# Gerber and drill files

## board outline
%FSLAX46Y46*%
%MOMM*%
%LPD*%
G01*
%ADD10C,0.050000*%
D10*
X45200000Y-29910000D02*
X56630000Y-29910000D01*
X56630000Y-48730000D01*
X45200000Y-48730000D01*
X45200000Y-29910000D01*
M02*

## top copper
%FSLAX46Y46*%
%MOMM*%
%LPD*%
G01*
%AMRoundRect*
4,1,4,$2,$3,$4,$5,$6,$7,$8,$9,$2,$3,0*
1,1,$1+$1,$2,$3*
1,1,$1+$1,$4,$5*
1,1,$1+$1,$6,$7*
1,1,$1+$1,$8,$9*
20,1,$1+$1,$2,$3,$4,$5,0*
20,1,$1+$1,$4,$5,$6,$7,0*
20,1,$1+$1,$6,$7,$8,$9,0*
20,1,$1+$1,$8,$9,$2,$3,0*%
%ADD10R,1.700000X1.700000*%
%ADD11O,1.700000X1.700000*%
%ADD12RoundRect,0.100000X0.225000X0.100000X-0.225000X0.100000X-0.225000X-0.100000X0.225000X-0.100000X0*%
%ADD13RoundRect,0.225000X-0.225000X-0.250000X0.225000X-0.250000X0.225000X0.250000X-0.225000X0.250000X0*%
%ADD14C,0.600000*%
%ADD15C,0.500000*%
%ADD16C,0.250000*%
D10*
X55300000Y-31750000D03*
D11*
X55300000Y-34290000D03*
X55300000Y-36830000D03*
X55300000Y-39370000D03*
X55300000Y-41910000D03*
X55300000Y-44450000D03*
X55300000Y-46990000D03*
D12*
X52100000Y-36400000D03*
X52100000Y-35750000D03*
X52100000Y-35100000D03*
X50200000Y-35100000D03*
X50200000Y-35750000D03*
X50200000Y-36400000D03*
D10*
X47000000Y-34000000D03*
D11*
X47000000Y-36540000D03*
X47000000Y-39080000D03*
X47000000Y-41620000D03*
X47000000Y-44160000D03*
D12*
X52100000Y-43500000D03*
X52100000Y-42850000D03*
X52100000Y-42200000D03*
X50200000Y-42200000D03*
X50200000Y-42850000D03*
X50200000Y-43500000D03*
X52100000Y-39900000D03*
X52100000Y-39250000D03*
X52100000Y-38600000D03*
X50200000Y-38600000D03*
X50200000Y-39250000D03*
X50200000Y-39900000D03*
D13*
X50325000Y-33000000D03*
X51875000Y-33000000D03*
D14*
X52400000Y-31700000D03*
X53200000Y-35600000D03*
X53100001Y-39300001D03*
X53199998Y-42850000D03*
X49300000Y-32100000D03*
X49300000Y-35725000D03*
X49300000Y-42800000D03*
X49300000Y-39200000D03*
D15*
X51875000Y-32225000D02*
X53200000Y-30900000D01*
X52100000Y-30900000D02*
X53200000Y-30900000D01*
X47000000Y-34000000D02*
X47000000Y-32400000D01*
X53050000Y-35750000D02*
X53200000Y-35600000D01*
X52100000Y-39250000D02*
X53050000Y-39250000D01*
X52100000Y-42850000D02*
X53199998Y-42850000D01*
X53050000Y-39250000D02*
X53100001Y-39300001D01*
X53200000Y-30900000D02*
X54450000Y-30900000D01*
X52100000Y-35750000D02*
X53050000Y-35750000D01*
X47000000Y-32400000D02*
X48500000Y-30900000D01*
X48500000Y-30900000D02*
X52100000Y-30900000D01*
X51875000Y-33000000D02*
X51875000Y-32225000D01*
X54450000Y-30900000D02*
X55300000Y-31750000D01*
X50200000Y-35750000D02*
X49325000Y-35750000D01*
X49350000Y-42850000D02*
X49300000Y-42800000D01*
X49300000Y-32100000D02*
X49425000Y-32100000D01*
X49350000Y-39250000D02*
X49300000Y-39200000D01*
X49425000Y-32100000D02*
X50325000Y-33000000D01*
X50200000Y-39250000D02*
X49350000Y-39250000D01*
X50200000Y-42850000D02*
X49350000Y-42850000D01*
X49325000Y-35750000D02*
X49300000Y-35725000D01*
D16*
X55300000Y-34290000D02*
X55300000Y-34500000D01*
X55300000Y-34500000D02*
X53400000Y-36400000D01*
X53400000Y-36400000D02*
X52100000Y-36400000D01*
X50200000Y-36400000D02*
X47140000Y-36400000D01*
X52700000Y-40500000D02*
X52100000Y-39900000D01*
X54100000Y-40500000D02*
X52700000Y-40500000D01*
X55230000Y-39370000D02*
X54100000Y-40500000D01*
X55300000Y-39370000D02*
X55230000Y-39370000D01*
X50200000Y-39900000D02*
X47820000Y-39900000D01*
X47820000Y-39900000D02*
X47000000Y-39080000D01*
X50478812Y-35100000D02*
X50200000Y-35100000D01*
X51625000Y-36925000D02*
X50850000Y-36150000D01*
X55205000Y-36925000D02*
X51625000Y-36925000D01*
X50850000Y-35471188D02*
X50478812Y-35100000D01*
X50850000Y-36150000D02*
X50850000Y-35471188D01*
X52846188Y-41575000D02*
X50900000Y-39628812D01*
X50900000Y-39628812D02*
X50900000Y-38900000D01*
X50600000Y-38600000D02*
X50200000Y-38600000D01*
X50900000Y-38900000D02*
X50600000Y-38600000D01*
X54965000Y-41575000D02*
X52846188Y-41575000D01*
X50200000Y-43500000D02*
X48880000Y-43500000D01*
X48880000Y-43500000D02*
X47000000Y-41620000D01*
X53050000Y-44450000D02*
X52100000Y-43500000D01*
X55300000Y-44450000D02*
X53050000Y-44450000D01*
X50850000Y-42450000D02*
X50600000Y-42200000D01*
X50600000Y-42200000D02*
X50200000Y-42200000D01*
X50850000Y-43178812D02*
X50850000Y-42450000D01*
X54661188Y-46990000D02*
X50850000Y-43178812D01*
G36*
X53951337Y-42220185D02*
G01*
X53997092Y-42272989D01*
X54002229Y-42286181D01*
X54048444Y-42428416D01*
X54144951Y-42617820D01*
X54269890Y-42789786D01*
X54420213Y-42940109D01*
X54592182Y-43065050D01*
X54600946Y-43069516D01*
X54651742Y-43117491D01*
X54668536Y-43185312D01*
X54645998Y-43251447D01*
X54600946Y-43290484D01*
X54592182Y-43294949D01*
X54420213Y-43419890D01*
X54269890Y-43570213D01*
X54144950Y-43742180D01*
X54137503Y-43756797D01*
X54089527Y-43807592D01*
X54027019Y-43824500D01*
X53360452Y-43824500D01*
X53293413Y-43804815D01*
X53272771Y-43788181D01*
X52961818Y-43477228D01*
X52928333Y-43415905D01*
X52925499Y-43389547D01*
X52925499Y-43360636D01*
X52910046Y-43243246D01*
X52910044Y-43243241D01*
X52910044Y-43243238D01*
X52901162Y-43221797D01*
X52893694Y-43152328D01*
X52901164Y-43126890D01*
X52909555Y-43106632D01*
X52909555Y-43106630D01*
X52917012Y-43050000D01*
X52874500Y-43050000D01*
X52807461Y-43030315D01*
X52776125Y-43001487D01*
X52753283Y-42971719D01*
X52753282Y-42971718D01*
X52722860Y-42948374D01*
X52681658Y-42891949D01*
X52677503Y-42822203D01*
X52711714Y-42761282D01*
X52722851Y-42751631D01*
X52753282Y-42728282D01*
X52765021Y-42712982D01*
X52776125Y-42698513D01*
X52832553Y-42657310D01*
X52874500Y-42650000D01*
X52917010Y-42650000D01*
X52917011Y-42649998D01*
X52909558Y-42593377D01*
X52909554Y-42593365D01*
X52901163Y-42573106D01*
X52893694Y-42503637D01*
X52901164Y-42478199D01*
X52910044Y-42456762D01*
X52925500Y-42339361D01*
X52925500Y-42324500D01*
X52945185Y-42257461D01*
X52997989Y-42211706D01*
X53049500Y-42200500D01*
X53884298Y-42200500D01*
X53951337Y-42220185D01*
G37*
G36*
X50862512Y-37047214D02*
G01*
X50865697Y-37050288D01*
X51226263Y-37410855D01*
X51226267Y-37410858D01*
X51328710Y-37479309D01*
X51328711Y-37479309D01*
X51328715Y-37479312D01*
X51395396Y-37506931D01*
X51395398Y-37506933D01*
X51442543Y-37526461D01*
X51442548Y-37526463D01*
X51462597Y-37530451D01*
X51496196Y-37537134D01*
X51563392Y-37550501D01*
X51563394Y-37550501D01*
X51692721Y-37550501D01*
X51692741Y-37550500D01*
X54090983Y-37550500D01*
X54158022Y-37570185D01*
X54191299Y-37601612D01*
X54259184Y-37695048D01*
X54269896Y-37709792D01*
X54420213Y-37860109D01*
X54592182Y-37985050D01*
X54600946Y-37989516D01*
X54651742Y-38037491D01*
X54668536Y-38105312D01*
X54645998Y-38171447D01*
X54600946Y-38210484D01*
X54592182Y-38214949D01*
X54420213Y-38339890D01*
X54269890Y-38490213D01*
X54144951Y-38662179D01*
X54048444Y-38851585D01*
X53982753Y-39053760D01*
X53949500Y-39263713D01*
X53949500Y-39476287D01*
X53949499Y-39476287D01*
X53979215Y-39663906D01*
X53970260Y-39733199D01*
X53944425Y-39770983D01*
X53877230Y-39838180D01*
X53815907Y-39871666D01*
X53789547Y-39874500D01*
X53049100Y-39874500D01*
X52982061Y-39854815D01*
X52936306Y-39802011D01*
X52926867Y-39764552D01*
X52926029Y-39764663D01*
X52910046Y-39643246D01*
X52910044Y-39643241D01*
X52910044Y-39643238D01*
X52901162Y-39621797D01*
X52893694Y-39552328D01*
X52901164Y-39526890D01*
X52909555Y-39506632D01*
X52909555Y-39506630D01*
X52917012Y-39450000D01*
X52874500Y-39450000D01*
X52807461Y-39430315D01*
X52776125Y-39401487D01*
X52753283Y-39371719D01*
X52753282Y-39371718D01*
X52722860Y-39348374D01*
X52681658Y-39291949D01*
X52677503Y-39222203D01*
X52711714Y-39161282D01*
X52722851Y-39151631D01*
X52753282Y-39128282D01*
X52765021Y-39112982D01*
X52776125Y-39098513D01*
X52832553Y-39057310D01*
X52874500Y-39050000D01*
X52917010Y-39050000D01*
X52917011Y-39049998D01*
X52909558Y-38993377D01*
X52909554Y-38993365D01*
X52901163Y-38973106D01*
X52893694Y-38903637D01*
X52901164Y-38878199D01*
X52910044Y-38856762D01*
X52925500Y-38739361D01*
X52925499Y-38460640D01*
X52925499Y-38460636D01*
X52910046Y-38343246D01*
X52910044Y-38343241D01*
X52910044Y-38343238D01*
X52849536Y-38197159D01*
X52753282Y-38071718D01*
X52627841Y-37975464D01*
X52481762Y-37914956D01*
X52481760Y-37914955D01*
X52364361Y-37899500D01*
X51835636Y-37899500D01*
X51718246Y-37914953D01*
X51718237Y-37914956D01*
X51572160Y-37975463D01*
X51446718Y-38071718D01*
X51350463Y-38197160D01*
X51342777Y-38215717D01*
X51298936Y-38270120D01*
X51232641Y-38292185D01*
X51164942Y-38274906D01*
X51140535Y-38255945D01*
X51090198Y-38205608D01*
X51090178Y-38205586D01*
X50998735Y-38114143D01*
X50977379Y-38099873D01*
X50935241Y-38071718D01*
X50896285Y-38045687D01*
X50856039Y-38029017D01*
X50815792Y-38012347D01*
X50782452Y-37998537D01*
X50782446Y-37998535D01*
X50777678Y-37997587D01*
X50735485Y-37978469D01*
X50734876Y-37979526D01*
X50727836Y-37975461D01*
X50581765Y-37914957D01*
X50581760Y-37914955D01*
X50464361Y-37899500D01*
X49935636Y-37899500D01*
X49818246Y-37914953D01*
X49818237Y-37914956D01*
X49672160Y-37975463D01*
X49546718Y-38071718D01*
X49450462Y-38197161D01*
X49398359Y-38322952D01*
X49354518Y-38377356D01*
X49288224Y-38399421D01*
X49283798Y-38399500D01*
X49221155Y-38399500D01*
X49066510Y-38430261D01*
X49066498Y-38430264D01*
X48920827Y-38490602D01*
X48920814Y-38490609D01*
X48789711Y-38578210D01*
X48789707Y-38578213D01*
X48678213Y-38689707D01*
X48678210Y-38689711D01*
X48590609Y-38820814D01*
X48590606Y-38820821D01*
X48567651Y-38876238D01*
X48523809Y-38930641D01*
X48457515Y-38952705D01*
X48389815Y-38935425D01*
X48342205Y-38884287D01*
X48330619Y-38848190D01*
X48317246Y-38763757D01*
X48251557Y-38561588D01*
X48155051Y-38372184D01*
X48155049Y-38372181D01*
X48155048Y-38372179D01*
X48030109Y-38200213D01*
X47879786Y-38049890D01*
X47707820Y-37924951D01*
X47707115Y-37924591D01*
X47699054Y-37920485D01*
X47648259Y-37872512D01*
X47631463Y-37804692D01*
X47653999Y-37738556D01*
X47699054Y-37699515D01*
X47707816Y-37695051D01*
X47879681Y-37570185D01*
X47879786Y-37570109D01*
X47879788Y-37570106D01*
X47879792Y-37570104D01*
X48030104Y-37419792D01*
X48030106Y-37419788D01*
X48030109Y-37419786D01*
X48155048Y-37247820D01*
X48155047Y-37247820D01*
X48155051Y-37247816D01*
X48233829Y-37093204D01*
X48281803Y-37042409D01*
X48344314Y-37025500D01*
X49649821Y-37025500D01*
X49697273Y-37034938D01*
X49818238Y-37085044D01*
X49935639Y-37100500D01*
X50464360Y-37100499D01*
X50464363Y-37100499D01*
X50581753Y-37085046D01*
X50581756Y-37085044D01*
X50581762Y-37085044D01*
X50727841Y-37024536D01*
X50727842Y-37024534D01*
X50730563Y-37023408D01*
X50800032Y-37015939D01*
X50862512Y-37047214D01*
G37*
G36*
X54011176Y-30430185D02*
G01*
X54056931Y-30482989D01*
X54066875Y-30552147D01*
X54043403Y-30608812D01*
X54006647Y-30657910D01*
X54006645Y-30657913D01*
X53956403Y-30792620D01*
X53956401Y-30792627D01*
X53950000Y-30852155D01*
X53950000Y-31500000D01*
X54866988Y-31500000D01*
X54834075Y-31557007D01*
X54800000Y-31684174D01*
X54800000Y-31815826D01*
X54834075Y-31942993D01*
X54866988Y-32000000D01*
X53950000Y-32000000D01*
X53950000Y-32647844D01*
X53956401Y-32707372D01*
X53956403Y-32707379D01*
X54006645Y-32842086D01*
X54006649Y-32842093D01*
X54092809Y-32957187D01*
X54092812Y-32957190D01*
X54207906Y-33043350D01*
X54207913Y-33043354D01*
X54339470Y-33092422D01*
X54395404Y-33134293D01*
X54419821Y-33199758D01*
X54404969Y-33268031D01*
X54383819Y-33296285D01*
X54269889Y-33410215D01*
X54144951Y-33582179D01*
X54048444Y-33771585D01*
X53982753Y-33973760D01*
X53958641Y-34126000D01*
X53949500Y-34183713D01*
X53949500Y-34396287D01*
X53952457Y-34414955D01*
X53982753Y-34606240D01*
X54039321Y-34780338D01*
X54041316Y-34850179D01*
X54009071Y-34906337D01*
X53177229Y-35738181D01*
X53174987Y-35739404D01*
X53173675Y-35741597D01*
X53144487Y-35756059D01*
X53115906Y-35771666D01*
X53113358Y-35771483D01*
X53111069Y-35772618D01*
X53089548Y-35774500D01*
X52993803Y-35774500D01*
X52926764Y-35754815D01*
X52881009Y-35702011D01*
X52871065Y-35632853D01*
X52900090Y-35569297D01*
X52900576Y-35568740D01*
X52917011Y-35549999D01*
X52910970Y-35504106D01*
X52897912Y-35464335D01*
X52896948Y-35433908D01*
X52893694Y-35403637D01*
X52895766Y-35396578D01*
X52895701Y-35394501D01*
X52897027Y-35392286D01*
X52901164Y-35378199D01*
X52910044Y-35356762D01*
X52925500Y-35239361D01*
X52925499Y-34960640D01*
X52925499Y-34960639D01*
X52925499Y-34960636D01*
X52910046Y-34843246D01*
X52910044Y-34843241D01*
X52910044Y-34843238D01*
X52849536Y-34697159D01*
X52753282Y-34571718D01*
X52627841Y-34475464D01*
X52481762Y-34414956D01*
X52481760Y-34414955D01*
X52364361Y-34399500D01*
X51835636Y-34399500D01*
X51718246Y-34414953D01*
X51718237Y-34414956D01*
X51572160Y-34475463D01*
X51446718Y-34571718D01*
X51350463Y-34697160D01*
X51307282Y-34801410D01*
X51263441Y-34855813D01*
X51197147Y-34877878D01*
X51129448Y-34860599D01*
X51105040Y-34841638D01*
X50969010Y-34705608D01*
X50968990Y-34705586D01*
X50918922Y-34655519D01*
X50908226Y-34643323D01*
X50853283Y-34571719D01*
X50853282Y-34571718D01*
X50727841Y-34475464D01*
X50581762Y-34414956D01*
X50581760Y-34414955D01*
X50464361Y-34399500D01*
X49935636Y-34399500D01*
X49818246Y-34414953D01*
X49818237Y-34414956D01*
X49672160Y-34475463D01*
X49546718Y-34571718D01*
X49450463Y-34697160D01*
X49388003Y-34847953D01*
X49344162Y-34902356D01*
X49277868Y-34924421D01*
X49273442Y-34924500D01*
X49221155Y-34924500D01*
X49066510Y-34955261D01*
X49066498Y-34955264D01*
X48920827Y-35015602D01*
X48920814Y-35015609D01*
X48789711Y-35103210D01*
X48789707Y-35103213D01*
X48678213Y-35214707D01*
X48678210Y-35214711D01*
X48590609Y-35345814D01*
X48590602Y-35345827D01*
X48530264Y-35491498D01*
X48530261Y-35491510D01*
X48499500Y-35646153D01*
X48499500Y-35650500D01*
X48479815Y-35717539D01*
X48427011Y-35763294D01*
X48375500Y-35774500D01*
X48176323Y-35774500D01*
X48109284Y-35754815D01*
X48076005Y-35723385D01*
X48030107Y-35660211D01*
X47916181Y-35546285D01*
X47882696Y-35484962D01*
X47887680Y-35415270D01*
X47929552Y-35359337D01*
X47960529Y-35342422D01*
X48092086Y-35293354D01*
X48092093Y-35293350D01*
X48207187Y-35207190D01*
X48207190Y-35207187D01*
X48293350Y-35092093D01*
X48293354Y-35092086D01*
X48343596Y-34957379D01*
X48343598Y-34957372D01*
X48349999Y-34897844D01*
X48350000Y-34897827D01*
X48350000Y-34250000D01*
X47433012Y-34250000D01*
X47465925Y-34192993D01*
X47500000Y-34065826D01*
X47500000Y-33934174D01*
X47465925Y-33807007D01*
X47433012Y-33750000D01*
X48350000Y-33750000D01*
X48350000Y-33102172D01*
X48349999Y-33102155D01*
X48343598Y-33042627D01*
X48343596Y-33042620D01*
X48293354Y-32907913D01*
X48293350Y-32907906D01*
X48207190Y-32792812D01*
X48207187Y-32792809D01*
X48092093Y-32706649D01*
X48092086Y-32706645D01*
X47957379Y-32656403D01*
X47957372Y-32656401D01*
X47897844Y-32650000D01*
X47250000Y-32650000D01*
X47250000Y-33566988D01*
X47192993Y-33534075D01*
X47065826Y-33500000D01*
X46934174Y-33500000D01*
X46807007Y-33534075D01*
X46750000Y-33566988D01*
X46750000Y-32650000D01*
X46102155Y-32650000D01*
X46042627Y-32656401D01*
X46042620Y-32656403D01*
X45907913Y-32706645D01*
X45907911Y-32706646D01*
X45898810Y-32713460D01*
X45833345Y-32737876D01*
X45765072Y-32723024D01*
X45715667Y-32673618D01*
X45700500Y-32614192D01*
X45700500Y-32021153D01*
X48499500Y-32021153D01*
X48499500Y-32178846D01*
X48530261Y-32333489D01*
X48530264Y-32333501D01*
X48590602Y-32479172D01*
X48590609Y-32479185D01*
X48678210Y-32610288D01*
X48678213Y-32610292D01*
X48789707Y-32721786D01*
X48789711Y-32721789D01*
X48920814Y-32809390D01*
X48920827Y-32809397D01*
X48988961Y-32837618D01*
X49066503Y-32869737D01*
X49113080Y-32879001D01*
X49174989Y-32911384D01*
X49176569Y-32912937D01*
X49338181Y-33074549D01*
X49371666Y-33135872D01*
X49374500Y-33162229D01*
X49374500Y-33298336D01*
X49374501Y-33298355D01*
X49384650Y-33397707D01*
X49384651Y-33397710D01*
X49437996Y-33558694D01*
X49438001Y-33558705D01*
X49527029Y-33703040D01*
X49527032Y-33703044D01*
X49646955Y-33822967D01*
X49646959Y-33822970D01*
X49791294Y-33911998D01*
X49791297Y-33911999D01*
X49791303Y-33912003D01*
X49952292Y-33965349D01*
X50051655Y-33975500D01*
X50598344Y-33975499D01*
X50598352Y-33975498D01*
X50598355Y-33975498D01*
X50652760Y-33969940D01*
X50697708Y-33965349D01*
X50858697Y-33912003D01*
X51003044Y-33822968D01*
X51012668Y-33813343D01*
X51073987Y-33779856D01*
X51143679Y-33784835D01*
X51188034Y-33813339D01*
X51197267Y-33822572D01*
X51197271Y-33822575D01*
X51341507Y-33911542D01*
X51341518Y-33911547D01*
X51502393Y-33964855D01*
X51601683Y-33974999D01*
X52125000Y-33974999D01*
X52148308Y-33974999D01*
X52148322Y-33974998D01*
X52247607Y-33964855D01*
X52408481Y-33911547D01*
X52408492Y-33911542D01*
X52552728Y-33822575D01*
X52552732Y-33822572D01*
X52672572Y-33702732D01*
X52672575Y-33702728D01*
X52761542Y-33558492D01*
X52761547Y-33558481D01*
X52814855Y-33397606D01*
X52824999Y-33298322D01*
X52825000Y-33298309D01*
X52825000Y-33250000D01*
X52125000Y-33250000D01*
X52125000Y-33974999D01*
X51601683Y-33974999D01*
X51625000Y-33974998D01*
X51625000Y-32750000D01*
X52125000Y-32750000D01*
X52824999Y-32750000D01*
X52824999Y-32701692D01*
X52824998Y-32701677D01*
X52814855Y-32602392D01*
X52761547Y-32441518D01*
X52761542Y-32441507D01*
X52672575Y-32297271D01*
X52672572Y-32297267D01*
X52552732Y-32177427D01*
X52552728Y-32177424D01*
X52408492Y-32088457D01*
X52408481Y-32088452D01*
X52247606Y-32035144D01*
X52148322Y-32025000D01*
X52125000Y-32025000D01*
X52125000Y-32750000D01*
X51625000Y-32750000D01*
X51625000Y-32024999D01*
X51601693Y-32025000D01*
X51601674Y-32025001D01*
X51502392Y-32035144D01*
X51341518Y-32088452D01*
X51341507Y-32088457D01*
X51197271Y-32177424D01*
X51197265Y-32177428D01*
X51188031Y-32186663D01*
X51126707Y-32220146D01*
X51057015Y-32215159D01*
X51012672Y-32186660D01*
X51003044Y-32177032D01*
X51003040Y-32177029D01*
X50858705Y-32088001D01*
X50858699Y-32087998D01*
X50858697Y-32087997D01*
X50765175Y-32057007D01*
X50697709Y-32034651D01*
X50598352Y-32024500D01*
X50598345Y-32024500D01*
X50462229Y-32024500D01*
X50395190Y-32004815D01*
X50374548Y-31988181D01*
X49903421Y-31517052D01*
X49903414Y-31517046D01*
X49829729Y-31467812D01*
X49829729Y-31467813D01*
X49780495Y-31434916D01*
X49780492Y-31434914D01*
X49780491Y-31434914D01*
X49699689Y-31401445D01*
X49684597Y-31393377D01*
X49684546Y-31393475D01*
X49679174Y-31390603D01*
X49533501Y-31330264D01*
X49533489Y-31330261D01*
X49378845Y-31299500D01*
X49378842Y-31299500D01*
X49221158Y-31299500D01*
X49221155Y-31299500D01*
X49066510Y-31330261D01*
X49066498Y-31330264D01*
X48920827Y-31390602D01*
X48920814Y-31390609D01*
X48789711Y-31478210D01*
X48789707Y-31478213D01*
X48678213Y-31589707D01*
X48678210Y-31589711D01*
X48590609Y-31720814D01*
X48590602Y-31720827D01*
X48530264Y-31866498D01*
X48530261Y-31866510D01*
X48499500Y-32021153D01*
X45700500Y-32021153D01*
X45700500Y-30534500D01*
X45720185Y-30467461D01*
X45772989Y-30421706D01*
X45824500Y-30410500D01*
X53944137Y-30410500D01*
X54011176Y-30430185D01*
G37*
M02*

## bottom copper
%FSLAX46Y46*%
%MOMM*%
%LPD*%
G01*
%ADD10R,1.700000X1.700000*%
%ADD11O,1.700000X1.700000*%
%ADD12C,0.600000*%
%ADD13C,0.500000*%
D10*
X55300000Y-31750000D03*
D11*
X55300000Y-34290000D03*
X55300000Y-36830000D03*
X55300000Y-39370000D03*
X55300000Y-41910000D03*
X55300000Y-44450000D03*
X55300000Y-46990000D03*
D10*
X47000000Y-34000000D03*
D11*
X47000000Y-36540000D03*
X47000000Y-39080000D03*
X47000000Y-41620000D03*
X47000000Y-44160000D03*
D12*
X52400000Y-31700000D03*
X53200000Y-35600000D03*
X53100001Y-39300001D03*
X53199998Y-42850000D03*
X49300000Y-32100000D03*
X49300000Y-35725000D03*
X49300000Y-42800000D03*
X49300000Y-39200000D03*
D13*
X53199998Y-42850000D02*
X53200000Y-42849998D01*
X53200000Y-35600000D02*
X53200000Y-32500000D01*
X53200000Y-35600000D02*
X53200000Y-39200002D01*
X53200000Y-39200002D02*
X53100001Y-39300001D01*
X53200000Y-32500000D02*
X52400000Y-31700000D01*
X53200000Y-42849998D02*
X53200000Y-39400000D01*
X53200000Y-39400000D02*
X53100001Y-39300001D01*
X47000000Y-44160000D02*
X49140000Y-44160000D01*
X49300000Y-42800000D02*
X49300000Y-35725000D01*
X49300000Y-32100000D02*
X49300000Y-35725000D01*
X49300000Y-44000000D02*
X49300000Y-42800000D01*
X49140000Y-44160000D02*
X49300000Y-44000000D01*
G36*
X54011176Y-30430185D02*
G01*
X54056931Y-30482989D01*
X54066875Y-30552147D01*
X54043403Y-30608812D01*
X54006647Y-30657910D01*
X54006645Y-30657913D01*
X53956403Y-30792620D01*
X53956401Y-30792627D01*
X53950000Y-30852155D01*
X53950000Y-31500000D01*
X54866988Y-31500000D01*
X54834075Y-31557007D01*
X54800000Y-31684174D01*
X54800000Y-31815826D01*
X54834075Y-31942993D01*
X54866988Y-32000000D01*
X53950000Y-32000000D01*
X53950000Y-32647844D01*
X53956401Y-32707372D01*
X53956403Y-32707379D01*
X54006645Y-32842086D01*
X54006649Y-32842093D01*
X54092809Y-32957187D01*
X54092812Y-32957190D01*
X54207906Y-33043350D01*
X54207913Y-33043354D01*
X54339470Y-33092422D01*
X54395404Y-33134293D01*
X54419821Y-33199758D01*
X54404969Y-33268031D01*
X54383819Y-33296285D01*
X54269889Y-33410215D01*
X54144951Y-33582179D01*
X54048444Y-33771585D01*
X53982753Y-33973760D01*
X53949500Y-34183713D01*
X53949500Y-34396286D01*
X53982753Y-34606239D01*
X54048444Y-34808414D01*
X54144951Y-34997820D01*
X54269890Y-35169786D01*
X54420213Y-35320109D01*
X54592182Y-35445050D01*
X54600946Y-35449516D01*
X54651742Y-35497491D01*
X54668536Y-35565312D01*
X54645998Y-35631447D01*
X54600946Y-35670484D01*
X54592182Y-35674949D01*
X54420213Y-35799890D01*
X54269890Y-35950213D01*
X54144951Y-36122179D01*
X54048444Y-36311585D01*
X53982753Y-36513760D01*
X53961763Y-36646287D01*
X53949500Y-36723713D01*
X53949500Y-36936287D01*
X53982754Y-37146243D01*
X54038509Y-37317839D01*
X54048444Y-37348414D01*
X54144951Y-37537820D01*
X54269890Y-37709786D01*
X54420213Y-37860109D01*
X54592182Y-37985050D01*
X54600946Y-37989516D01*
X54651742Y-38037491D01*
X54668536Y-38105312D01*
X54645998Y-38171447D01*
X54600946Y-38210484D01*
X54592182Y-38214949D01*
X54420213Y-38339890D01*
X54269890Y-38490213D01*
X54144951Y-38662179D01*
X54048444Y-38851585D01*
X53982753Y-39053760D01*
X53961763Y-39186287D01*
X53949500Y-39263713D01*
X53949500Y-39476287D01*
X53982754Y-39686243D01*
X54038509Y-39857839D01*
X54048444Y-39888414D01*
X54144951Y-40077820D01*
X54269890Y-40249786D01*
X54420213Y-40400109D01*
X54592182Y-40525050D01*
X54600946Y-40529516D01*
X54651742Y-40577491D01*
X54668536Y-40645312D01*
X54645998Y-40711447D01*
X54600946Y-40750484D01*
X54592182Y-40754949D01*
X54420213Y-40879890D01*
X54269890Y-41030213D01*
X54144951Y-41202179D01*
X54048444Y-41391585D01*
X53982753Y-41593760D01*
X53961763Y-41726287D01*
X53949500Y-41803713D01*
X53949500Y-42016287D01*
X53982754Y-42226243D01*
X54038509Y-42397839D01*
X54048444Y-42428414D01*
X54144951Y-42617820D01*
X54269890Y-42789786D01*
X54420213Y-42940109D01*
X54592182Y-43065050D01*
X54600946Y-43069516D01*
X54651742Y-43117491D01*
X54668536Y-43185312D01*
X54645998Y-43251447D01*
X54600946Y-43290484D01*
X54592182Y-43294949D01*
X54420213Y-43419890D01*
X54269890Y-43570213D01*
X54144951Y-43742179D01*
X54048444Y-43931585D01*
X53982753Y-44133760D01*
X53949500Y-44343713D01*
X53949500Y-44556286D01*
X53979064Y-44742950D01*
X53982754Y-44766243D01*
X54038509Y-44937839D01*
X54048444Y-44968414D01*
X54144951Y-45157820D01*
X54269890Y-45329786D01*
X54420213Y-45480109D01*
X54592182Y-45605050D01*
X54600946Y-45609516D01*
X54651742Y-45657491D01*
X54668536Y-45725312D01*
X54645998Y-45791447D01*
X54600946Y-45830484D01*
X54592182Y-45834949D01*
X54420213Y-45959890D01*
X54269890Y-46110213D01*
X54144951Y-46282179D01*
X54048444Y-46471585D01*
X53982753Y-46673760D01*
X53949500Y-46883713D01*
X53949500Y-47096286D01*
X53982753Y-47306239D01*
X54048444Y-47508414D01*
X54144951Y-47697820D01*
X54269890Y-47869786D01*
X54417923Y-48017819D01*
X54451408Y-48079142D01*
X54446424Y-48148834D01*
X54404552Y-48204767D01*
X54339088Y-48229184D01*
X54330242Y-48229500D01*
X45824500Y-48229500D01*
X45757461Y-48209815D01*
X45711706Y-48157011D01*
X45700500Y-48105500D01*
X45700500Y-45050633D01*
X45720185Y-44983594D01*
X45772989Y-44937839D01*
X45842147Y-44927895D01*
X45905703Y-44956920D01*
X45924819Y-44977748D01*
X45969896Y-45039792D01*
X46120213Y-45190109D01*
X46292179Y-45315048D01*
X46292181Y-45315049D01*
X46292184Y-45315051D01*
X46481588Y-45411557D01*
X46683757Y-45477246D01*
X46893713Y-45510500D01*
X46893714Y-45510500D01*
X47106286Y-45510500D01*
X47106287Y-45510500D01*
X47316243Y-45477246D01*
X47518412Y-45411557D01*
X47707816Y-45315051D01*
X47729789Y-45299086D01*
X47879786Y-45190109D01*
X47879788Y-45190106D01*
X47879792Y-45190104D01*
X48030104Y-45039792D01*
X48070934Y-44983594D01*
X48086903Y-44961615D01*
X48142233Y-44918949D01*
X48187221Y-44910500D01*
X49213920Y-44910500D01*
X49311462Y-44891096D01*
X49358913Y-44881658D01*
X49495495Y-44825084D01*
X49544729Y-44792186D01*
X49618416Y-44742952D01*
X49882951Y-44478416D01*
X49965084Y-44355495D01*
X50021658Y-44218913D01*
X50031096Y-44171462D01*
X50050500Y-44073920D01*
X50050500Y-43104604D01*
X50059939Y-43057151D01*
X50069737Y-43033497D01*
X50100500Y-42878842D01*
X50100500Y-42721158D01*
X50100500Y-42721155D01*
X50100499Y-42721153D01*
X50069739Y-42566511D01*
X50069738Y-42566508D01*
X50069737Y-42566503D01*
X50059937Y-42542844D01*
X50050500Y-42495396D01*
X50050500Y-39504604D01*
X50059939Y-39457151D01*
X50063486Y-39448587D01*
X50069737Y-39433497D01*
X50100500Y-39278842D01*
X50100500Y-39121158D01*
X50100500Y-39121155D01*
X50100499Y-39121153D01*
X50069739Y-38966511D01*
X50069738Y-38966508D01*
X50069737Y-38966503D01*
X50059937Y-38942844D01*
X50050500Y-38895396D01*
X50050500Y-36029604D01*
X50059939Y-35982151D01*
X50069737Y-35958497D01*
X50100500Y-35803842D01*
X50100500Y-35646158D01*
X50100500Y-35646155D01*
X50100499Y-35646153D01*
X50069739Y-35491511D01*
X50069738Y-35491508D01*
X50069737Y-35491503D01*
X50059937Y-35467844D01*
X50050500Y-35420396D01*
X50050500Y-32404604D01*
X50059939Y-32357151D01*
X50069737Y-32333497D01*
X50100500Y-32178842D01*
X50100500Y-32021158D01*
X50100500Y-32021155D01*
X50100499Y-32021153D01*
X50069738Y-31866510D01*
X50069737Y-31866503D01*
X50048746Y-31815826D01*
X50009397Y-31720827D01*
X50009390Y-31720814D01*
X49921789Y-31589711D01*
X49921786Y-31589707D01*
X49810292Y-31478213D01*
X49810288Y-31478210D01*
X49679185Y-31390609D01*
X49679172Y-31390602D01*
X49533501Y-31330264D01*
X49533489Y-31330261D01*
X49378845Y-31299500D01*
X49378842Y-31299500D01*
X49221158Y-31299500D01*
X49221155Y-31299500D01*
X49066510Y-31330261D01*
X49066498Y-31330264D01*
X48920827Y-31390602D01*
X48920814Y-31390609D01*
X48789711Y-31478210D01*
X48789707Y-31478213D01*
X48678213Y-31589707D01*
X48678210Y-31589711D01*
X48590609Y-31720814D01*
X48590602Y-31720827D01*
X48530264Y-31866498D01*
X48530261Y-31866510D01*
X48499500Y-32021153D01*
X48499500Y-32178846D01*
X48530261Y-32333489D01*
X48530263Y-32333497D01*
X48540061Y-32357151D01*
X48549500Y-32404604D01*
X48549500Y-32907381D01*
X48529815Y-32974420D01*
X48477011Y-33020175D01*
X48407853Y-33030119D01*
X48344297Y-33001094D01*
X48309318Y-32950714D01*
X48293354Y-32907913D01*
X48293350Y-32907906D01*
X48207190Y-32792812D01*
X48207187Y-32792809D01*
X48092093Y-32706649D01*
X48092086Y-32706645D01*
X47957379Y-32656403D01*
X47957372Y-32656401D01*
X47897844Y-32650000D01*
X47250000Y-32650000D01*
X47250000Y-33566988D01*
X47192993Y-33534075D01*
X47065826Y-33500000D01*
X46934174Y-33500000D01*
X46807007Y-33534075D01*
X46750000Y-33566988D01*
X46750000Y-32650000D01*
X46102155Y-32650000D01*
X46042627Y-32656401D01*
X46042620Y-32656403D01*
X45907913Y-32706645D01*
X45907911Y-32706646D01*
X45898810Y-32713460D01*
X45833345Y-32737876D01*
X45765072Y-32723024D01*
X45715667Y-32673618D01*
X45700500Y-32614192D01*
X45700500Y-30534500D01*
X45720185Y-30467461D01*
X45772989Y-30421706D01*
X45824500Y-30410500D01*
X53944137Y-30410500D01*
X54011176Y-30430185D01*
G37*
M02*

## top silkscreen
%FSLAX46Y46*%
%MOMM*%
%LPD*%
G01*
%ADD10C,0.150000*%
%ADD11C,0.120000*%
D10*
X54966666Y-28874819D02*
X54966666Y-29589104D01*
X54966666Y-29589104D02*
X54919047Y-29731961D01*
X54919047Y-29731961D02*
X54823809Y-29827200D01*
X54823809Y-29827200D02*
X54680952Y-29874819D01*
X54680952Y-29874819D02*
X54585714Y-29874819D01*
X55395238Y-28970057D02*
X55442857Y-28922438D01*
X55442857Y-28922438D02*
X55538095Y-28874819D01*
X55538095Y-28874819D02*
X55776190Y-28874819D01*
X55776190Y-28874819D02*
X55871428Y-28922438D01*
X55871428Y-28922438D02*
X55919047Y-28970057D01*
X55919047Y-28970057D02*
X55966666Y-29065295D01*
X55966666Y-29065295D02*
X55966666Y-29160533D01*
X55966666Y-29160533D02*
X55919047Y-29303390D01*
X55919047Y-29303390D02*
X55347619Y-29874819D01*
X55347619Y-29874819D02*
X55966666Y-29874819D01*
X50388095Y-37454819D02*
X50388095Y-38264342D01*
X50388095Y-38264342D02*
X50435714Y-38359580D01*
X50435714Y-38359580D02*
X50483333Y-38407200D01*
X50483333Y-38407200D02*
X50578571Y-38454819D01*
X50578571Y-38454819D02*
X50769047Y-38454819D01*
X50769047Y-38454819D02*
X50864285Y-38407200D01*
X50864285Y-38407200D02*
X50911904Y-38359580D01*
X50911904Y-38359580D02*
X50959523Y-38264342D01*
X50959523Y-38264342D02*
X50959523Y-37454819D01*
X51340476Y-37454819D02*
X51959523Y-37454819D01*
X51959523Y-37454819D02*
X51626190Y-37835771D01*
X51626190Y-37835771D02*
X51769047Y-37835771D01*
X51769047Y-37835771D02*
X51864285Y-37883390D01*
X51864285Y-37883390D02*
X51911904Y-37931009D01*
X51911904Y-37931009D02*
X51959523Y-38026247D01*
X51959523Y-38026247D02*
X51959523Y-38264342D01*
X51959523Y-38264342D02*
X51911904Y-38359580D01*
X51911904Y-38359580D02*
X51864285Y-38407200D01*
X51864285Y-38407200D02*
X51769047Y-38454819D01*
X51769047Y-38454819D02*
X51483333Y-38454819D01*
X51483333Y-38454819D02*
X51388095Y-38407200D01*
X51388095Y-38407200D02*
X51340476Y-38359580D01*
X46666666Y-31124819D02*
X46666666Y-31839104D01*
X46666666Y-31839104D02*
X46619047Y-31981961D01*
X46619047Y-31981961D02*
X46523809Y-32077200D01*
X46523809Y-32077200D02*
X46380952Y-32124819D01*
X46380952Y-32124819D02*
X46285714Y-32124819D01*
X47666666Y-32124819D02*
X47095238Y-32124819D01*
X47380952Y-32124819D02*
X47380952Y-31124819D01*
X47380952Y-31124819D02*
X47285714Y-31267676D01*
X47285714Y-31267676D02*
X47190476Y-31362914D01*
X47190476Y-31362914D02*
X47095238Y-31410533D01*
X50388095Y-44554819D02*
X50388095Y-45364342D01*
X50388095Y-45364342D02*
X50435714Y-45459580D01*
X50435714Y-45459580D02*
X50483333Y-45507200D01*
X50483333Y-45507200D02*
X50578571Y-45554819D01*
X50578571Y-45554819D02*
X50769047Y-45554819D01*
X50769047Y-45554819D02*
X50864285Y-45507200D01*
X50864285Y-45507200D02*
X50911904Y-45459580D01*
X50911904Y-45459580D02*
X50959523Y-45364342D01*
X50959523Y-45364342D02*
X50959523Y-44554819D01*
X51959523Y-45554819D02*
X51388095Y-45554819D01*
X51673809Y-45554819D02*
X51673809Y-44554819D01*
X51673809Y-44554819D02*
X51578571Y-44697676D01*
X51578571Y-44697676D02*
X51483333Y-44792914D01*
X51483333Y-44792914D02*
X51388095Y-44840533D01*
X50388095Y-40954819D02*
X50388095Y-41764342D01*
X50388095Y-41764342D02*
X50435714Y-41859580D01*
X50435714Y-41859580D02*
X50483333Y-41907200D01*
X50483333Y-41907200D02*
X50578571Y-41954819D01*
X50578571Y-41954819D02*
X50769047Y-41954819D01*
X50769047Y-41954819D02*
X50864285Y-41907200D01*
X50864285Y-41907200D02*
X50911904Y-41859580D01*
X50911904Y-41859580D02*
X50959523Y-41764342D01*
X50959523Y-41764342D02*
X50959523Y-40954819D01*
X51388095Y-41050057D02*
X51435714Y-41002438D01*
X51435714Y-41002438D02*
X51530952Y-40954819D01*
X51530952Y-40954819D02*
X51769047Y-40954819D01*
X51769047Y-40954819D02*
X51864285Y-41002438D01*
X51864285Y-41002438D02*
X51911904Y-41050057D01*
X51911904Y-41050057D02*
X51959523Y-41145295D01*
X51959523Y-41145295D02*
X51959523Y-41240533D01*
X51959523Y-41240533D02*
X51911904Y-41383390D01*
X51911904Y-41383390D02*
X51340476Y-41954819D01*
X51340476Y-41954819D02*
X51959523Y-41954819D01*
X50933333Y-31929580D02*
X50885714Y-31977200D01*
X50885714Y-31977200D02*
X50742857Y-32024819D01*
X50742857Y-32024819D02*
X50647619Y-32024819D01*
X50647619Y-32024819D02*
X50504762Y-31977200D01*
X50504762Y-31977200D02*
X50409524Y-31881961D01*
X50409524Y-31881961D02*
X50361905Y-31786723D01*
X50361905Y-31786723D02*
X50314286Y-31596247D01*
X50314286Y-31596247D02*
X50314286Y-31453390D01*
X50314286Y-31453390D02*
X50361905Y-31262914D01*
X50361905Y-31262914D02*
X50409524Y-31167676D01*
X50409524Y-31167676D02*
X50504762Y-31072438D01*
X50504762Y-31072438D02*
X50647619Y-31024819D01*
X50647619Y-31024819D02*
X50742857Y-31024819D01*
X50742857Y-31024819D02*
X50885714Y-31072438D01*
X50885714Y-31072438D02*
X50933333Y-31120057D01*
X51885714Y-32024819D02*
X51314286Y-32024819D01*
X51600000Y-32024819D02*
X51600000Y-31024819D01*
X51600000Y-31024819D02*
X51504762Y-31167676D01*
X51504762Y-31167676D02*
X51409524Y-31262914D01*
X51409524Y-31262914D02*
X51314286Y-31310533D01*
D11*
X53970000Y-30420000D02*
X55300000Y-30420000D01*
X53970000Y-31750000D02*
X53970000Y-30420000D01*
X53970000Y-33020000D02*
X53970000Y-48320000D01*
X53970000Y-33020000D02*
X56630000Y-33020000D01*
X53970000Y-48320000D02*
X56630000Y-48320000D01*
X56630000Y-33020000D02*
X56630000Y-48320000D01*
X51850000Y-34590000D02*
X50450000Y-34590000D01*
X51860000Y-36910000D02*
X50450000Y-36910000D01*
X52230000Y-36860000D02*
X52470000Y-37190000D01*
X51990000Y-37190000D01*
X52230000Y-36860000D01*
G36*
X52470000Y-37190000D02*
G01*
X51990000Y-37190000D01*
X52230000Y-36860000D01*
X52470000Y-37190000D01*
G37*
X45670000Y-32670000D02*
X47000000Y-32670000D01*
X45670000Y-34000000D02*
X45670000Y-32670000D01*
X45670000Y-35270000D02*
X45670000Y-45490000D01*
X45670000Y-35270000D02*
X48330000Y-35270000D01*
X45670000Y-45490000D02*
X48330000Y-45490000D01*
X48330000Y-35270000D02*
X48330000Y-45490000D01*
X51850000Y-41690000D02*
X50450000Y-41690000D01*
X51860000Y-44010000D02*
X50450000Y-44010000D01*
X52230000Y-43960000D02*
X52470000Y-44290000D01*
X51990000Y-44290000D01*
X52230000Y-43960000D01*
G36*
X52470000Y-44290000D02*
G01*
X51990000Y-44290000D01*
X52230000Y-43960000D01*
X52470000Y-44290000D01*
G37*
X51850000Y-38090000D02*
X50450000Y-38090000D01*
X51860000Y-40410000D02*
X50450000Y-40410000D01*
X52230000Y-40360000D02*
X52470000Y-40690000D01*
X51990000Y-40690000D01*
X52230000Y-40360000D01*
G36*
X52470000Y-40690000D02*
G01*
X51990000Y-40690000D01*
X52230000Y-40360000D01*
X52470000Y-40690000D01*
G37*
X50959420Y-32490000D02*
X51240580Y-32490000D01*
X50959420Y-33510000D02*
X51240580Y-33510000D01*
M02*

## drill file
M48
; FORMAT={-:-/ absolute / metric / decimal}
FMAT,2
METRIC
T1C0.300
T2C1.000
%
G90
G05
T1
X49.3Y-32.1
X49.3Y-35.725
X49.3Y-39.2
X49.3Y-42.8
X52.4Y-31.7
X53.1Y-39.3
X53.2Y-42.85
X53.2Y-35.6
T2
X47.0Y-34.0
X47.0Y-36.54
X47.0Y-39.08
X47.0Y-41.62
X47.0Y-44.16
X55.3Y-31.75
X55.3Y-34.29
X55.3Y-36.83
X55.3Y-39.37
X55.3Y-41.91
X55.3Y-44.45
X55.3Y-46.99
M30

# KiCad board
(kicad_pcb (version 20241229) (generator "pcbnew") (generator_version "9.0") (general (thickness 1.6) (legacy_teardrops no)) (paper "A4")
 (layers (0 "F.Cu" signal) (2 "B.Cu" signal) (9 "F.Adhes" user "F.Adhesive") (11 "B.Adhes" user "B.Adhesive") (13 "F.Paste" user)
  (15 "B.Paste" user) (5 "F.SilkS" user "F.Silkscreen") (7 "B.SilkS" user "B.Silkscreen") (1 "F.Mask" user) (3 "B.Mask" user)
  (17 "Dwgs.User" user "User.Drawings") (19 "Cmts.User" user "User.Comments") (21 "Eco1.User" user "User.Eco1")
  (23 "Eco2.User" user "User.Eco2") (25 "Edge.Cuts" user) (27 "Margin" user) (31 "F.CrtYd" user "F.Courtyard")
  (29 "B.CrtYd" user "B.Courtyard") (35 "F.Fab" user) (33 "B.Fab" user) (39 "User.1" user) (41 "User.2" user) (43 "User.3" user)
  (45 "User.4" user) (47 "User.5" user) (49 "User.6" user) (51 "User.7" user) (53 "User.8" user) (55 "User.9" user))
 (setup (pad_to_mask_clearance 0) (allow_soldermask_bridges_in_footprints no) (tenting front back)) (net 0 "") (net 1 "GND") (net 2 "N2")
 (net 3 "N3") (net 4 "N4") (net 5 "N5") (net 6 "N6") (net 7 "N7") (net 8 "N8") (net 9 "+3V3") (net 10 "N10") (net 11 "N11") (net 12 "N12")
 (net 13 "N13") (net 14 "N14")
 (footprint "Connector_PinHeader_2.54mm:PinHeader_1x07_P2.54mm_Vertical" (layer "F.Cu") (at 55.3 31.75)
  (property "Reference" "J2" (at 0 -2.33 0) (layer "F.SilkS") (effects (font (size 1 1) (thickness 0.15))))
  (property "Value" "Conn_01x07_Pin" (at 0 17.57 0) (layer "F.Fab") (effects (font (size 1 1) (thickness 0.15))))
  (fp_line (start -1.33 -1.33) (end 0 -1.33) (stroke (width 0.12) (type solid)) (layer "F.SilkS"))
  (fp_line (start -1.33 0) (end -1.33 -1.33) (stroke (width 0.12) (type solid)) (layer "F.SilkS"))
  (fp_line (start -1.33 1.27) (end -1.33 16.57) (stroke (width 0.12) (type solid)) (layer "F.SilkS"))
  (fp_line (start -1.33 1.27) (end 1.33 1.27) (stroke (width 0.12) (type solid)) (layer "F.SilkS"))
  (fp_line (start -1.33 16.57) (end 1.33 16.57) (stroke (width 0.12) (type solid)) (layer "F.SilkS"))
  (fp_line (start 1.33 1.27) (end 1.33 16.57) (stroke (width 0.12) (type solid)) (layer "F.SilkS"))
  (pad "1" thru_hole rect (at 0 0) (size 1.7 1.7) (drill 1) (layers "*.Cu" "*.Mask") (remove_unused_layers no) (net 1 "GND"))
  (pad "2" thru_hole oval (at 0 2.54) (size 1.7 1.7) (drill 1) (layers "*.Cu" "*.Mask") (remove_unused_layers no) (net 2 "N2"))
  (pad "3" thru_hole oval (at 0 5.08) (size 1.7 1.7) (drill 1) (layers "*.Cu" "*.Mask") (remove_unused_layers no) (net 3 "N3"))
  (pad "4" thru_hole oval (at 0 7.62) (size 1.7 1.7) (drill 1) (layers "*.Cu" "*.Mask") (remove_unused_layers no) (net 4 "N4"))
  (pad "5" thru_hole oval (at 0 10.16) (size 1.7 1.7) (drill 1) (layers "*.Cu" "*.Mask") (remove_unused_layers no) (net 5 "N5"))
  (pad "6" thru_hole oval (at 0 12.7) (size 1.7 1.7) (drill 1) (layers "*.Cu" "*.Mask") (remove_unused_layers no) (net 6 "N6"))
  (pad "7" thru_hole oval (at 0 15.24) (size 1.7 1.7) (drill 1) (layers "*.Cu" "*.Mask") (remove_unused_layers no) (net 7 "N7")))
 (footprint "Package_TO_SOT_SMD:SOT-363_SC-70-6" (layer "F.Cu") (at 51.15 35.75 180)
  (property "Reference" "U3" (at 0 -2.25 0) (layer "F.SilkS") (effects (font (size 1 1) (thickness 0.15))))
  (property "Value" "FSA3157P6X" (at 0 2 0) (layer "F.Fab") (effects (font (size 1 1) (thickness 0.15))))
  (fp_line (start -0.7 1.16) (end 0.7 1.16) (stroke (width 0.12) (type solid)) (layer "F.SilkS"))
  (fp_line (start -0.71 -1.16) (end 0.7 -1.16) (stroke (width 0.12) (type solid)) (layer "F.SilkS"))
  (fp_poly
   (pts (xy -1.08 -1.11) (xy -1.32 -1.44) (xy -0.84 -1.44) (xy -1.08 -1.11)) (stroke (width 0.12) (type solid)) (fill yes) (layer "F.SilkS"))
  (pad "1" smd roundrect (at -0.95 -0.65 180) (size 0.65 0.4) (layers "F.Cu" "F.Mask" "F.Paste") (roundrect_rratio 0.25) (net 2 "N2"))
  (pad "2" smd roundrect (at -0.95 0 180) (size 0.65 0.4) (layers "F.Cu" "F.Mask" "F.Paste") (roundrect_rratio 0.25) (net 1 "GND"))
  (pad "3" smd roundrect (at -0.95 0.65 180) (size 0.65 0.4) (layers "F.Cu" "F.Mask" "F.Paste") (roundrect_rratio 0.25) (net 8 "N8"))
  (pad "4" smd roundrect (at 0.95 0.65 180) (size 0.65 0.4) (layers "F.Cu" "F.Mask" "F.Paste") (roundrect_rratio 0.25) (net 3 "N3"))
  (pad "5" smd roundrect (at 0.95 0 180) (size 0.65 0.4) (layers "F.Cu" "F.Mask" "F.Paste") (roundrect_rratio 0.25) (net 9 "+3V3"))
  (pad "6" smd roundrect (at 0.95 -0.65 180) (size 0.65 0.4) (layers "F.Cu" "F.Mask" "F.Paste") (roundrect_rratio 0.25) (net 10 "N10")))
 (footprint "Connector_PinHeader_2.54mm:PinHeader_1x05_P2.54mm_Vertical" (layer "F.Cu") (at 47 34)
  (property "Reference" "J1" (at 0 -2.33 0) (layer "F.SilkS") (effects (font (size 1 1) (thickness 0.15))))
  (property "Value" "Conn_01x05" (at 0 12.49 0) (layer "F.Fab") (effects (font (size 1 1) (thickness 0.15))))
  (fp_line (start -1.33 -1.33) (end 0 -1.33) (stroke (width 0.12) (type solid)) (layer "F.SilkS"))
  (fp_line (start -1.33 0) (end -1.33 -1.33) (stroke (width 0.12) (type solid)) (layer "F.SilkS"))
  (fp_line (start -1.33 1.27) (end -1.33 11.49) (stroke (width 0.12) (type solid)) (layer "F.SilkS"))
  (fp_line (start -1.33 1.27) (end 1.33 1.27) (stroke (width 0.12) (type solid)) (layer "F.SilkS"))
  (fp_line (start -1.33 11.49) (end 1.33 11.49) (stroke (width 0.12) (type solid)) (layer "F.SilkS"))
  (fp_line (start 1.33 1.27) (end 1.33 11.49) (stroke (width 0.12) (type solid)) (layer "F.SilkS"))
  (pad "1" thru_hole rect (at 0 0) (size 1.7 1.7) (drill 1) (layers "*.Cu" "*.Mask") (remove_unused_layers no) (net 1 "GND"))
  (pad "2" thru_hole oval (at 0 2.54) (size 1.7 1.7) (drill 1) (layers "*.Cu" "*.Mask") (remove_unused_layers no) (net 10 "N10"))
  (pad "3" thru_hole oval (at 0 5.08) (size 1.7 1.7) (drill 1) (layers "*.Cu" "*.Mask") (remove_unused_layers no) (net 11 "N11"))
  (pad "4" thru_hole oval (at 0 7.62) (size 1.7 1.7) (drill 1) (layers "*.Cu" "*.Mask") (remove_unused_layers no) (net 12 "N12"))
  (pad "5" thru_hole oval (at 0 10.16) (size 1.7 1.7) (drill 1) (layers "*.Cu" "*.Mask") (remove_unused_layers no) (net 9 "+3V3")))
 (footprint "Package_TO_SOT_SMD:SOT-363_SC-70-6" (layer "F.Cu") (at 51.15 42.85 180)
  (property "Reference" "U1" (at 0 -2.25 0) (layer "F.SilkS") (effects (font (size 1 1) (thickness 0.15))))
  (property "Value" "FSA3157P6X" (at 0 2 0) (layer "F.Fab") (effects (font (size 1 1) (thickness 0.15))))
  (fp_line (start -0.7 1.16) (end 0.7 1.16) (stroke (width 0.12) (type solid)) (layer "F.SilkS"))
  (fp_line (start -0.71 -1.16) (end 0.7 -1.16) (stroke (width 0.12) (type solid)) (layer "F.SilkS"))
  (fp_poly
   (pts (xy -1.08 -1.11) (xy -1.32 -1.44) (xy -0.84 -1.44) (xy -1.08 -1.11)) (stroke (width 0.12) (type solid)) (fill yes) (layer "F.SilkS"))
  (pad "1" smd roundrect (at -0.95 -0.65 180) (size 0.65 0.4) (layers "F.Cu" "F.Mask" "F.Paste") (roundrect_rratio 0.25) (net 6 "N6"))
  (pad "2" smd roundrect (at -0.95 0 180) (size 0.65 0.4) (layers "F.Cu" "F.Mask" "F.Paste") (roundrect_rratio 0.25) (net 1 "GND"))
  (pad "3" smd roundrect (at -0.95 0.65 180) (size 0.65 0.4) (layers "F.Cu" "F.Mask" "F.Paste") (roundrect_rratio 0.25) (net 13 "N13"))
  (pad "4" smd roundrect (at 0.95 0.65 180) (size 0.65 0.4) (layers "F.Cu" "F.Mask" "F.Paste") (roundrect_rratio 0.25) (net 7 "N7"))
  (pad "5" smd roundrect (at 0.95 0 180) (size 0.65 0.4) (layers "F.Cu" "F.Mask" "F.Paste") (roundrect_rratio 0.25) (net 9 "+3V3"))
  (pad "6" smd roundrect (at 0.95 -0.65 180) (size 0.65 0.4) (layers "F.Cu" "F.Mask" "F.Paste") (roundrect_rratio 0.25) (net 12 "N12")))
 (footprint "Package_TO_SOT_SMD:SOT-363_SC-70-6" (layer "F.Cu") (at 51.15 39.25 180)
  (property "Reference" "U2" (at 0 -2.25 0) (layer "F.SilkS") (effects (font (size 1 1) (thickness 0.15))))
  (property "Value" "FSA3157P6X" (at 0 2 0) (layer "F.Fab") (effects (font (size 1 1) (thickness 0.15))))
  (fp_line (start -0.7 1.16) (end 0.7 1.16) (stroke (width 0.12) (type solid)) (layer "F.SilkS"))
  (fp_line (start -0.71 -1.16) (end 0.7 -1.16) (stroke (width 0.12) (type solid)) (layer "F.SilkS"))
  (fp_poly
   (pts (xy -1.08 -1.11) (xy -1.32 -1.44) (xy -0.84 -1.44) (xy -1.08 -1.11)) (stroke (width 0.12) (type solid)) (fill yes) (layer "F.SilkS"))
  (pad "1" smd roundrect (at -0.95 -0.65 180) (size 0.65 0.4) (layers "F.Cu" "F.Mask" "F.Paste") (roundrect_rratio 0.25) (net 4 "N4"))
  (pad "2" smd roundrect (at -0.95 0 180) (size 0.65 0.4) (layers "F.Cu" "F.Mask" "F.Paste") (roundrect_rratio 0.25) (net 1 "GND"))
  (pad "3" smd roundrect (at -0.95 0.65 180) (size 0.65 0.4) (layers "F.Cu" "F.Mask" "F.Paste") (roundrect_rratio 0.25) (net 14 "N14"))
  (pad "4" smd roundrect (at 0.95 0.65 180) (size 0.65 0.4) (layers "F.Cu" "F.Mask" "F.Paste") (roundrect_rratio 0.25) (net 5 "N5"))
  (pad "5" smd roundrect (at 0.95 0 180) (size 0.65 0.4) (layers "F.Cu" "F.Mask" "F.Paste") (roundrect_rratio 0.25) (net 9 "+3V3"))
  (pad "6" smd roundrect (at 0.95 -0.65 180) (size 0.65 0.4) (layers "F.Cu" "F.Mask" "F.Paste") (roundrect_rratio 0.25) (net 11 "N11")))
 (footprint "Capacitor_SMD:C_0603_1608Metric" (layer "F.Cu") (at 51.1 33)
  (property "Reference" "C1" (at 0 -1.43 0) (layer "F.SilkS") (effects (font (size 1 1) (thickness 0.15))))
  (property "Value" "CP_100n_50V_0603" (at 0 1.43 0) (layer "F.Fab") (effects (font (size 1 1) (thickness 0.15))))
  (fp_line (start -0.14058 -0.51) (end 0.14058 -0.51) (stroke (width 0.12) (type solid)) (layer "F.SilkS"))
  (fp_line (start -0.14058 0.51) (end 0.14058 0.51) (stroke (width 0.12) (type solid)) (layer "F.SilkS"))
  (pad "1" smd roundrect (at -0.775 0) (size 0.9 0.95) (layers "F.Cu" "F.Mask" "F.Paste") (roundrect_rratio 0.25) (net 9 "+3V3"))
  (pad "2" smd roundrect (at 0.775 0) (size 0.9 0.95) (layers "F.Cu" "F.Mask" "F.Paste") (roundrect_rratio 0.25) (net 1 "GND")))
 (gr_rect (start 45.2 29.91) (end 56.63 48.73) (stroke (width 0.05) (type default)) (fill no) (layer "Edge.Cuts"))
 (segment (start 51.875 32.225) (end 53.2 30.9) (width 0.5) (layer "F.Cu") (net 1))
 (segment (start 52.1 30.9) (end 53.2 30.9) (width 0.5) (layer "F.Cu") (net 1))
 (segment (start 47 34) (end 47 32.4) (width 0.5) (layer "F.Cu") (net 1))
 (segment (start 53.05 35.75) (end 53.2 35.6) (width 0.5) (layer "F.Cu") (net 1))
 (segment (start 52.1 39.25) (end 53.05 39.25) (width 0.5) (layer "F.Cu") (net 1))
 (segment (start 52.1 42.85) (end 53.199998 42.85) (width 0.5) (layer "F.Cu") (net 1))
 (segment (start 53.05 39.25) (end 53.100001 39.300001) (width 0.5) (layer "F.Cu") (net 1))
 (segment (start 53.2 30.9) (end 54.45 30.9) (width 0.5) (layer "F.Cu") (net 1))
 (segment (start 52.1 35.75) (end 53.05 35.75) (width 0.5) (layer "F.Cu") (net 1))
 (segment (start 47 32.4) (end 48.5 30.9) (width 0.5) (layer "F.Cu") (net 1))
 (segment (start 48.5 30.9) (end 52.1 30.9) (width 0.5) (layer "F.Cu") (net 1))
 (segment (start 51.875 33) (end 51.875 32.225) (width 0.5) (layer "F.Cu") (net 1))
 (segment (start 54.45 30.9) (end 55.3 31.75) (width 0.5) (layer "F.Cu") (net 1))
 (via (at 52.4 31.7) (size 0.6) (drill 0.3) (layers "F.Cu" "B.Cu") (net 1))
 (via (at 53.2 35.6) (size 0.6) (drill 0.3) (layers "F.Cu" "B.Cu") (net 1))
 (via (at 53.100001 39.300001) (size 0.6) (drill 0.3) (layers "F.Cu" "B.Cu") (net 1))
 (via (at 53.199998 42.85) (size 0.6) (drill 0.3) (layers "F.Cu" "B.Cu") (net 1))
 (segment (start 53.199998 42.85) (end 53.2 42.849998) (width 0.5) (layer "B.Cu") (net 1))
 (segment (start 53.2 35.6) (end 53.2 32.5) (width 0.5) (layer "B.Cu") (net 1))
 (segment (start 53.2 35.6) (end 53.2 39.200002) (width 0.5) (layer "B.Cu") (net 1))
 (segment (start 53.2 39.200002) (end 53.100001 39.300001) (width 0.5) (layer "B.Cu") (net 1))
 (segment (start 53.2 32.5) (end 52.4 31.7) (width 0.5) (layer "B.Cu") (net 1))
 (segment (start 53.2 42.849998) (end 53.2 39.4) (width 0.5) (layer "B.Cu") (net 1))
 (segment (start 53.2 39.4) (end 53.100001 39.300001) (width 0.5) (layer "B.Cu") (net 1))
 (segment (start 50.2 35.75) (end 49.325 35.75) (width 0.5) (layer "F.Cu") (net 9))
 (segment (start 49.35 42.85) (end 49.3 42.8) (width 0.5) (layer "F.Cu") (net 9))
 (segment (start 49.3 32.1) (end 49.425 32.1) (width 0.5) (layer "F.Cu") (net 9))
 (segment (start 49.35 39.25) (end 49.3 39.2) (width 0.5) (layer "F.Cu") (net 9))
 (segment (start 49.425 32.1) (end 50.325 33) (width 0.5) (layer "F.Cu") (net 9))
 (segment (start 50.2 39.25) (end 49.35 39.25) (width 0.5) (layer "F.Cu") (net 9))
 (segment (start 50.2 42.85) (end 49.35 42.85) (width 0.5) (layer "F.Cu") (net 9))
 (segment (start 49.325 35.75) (end 49.3 35.725) (width 0.5) (layer "F.Cu") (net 9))
 (via (at 49.3 32.1) (size 0.6) (drill 0.3) (layers "F.Cu" "B.Cu") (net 9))
 (via (at 49.3 35.725) (size 0.6) (drill 0.3) (layers "F.Cu" "B.Cu") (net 9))
 (via (at 49.3 42.8) (size 0.6) (drill 0.3) (layers "F.Cu" "B.Cu") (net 9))
 (via (at 49.3 39.2) (size 0.6) (drill 0.3) (layers "F.Cu" "B.Cu") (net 9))
 (segment (start 47 44.16) (end 49.14 44.16) (width 0.5) (layer "B.Cu") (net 9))
 (segment (start 49.3 42.8) (end 49.3 35.725) (width 0.5) (layer "B.Cu") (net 9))
 (segment (start 49.3 32.1) (end 49.3 35.725) (width 0.5) (layer "B.Cu") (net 9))
 (segment (start 49.3 44) (end 49.3 42.8) (width 0.5) (layer "B.Cu") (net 9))
 (segment (start 49.14 44.16) (end 49.3 44) (width 0.5) (layer "B.Cu") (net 9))
 (segment (start 55.3 34.29) (end 55.3 34.5) (width 0.25) (layer "F.Cu") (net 2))
 (segment (start 55.3 34.5) (end 53.4 36.4) (width 0.25) (layer "F.Cu") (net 2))
 (segment (start 53.4 36.4) (end 52.1 36.4) (width 0.25) (layer "F.Cu") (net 2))
 (segment (start 50.2 36.4) (end 47.14 36.4) (width 0.25) (layer "F.Cu") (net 10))
 (segment (start 52.7 40.5) (end 52.1 39.9) (width 0.25) (layer "F.Cu") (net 4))
 (segment (start 54.1 40.5) (end 52.7 40.5) (width 0.25) (layer "F.Cu") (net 4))
 (segment (start 55.23 39.37) (end 54.1 40.5) (width 0.25) (layer "F.Cu") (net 4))
 (segment (start 55.3 39.37) (end 55.23 39.37) (width 0.25) (layer "F.Cu") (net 4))
 (segment (start 50.2 39.9) (end 47.82 39.9) (width 0.25) (layer "F.Cu") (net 11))
 (segment (start 47.82 39.9) (end 47 39.08) (width 0.25) (layer "F.Cu") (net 11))
 (segment (start 50.478812 35.1) (end 50.2 35.1) (width 0.25) (layer "F.Cu") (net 3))
 (segment (start 51.625 36.925) (end 50.85 36.15) (width 0.25) (layer "F.Cu") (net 3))
 (segment (start 55.205 36.925) (end 51.625 36.925) (width 0.25) (layer "F.Cu") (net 3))
 (segment (start 50.85 35.471188) (end 50.478812 35.1) (width 0.25) (layer "F.Cu") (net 3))
 (segment (start 50.85 36.15) (end 50.85 35.471188) (width 0.25) (layer "F.Cu") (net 3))
 (segment (start 52.846188 41.575) (end 50.9 39.628812) (width 0.25) (layer "F.Cu") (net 5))
 (segment (start 50.9 39.628812) (end 50.9 38.9) (width 0.25) (layer "F.Cu") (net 5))
 (segment (start 50.6 38.6) (end 50.2 38.6) (width 0.25) (layer "F.Cu") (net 5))
 (segment (start 50.9 38.9) (end 50.6 38.6) (width 0.25) (layer "F.Cu") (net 5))
 (segment (start 54.965 41.575) (end 52.846188 41.575) (width 0.25) (layer "F.Cu") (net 5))
 (segment (start 50.2 43.5) (end 48.88 43.5) (width 0.25) (layer "F.Cu") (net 12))
 (segment (start 48.88 43.5) (end 47 41.62) (width 0.25) (layer "F.Cu") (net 12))
 (segment (start 53.05 44.45) (end 52.1 43.5) (width 0.25) (layer "F.Cu") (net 6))
 (segment (start 55.3 44.45) (end 53.05 44.45) (width 0.25) (layer "F.Cu") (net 6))
 (segment (start 50.85 42.45) (end 50.6 42.2) (width 0.25) (layer "F.Cu") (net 7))
 (segment (start 50.6 42.2) (end 50.2 42.2) (width 0.25) (layer "F.Cu") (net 7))
 (segment (start 50.85 43.178812) (end 50.85 42.45) (width 0.25) (layer "F.Cu") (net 7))
 (segment (start 54.661188 46.99) (end 50.85 43.178812) (width 0.25) (layer "F.Cu") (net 7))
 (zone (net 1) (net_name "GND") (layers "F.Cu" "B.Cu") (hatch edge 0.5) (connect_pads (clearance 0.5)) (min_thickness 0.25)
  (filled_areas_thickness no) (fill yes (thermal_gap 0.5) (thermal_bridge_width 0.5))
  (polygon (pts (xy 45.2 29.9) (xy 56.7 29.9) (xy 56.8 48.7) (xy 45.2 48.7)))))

